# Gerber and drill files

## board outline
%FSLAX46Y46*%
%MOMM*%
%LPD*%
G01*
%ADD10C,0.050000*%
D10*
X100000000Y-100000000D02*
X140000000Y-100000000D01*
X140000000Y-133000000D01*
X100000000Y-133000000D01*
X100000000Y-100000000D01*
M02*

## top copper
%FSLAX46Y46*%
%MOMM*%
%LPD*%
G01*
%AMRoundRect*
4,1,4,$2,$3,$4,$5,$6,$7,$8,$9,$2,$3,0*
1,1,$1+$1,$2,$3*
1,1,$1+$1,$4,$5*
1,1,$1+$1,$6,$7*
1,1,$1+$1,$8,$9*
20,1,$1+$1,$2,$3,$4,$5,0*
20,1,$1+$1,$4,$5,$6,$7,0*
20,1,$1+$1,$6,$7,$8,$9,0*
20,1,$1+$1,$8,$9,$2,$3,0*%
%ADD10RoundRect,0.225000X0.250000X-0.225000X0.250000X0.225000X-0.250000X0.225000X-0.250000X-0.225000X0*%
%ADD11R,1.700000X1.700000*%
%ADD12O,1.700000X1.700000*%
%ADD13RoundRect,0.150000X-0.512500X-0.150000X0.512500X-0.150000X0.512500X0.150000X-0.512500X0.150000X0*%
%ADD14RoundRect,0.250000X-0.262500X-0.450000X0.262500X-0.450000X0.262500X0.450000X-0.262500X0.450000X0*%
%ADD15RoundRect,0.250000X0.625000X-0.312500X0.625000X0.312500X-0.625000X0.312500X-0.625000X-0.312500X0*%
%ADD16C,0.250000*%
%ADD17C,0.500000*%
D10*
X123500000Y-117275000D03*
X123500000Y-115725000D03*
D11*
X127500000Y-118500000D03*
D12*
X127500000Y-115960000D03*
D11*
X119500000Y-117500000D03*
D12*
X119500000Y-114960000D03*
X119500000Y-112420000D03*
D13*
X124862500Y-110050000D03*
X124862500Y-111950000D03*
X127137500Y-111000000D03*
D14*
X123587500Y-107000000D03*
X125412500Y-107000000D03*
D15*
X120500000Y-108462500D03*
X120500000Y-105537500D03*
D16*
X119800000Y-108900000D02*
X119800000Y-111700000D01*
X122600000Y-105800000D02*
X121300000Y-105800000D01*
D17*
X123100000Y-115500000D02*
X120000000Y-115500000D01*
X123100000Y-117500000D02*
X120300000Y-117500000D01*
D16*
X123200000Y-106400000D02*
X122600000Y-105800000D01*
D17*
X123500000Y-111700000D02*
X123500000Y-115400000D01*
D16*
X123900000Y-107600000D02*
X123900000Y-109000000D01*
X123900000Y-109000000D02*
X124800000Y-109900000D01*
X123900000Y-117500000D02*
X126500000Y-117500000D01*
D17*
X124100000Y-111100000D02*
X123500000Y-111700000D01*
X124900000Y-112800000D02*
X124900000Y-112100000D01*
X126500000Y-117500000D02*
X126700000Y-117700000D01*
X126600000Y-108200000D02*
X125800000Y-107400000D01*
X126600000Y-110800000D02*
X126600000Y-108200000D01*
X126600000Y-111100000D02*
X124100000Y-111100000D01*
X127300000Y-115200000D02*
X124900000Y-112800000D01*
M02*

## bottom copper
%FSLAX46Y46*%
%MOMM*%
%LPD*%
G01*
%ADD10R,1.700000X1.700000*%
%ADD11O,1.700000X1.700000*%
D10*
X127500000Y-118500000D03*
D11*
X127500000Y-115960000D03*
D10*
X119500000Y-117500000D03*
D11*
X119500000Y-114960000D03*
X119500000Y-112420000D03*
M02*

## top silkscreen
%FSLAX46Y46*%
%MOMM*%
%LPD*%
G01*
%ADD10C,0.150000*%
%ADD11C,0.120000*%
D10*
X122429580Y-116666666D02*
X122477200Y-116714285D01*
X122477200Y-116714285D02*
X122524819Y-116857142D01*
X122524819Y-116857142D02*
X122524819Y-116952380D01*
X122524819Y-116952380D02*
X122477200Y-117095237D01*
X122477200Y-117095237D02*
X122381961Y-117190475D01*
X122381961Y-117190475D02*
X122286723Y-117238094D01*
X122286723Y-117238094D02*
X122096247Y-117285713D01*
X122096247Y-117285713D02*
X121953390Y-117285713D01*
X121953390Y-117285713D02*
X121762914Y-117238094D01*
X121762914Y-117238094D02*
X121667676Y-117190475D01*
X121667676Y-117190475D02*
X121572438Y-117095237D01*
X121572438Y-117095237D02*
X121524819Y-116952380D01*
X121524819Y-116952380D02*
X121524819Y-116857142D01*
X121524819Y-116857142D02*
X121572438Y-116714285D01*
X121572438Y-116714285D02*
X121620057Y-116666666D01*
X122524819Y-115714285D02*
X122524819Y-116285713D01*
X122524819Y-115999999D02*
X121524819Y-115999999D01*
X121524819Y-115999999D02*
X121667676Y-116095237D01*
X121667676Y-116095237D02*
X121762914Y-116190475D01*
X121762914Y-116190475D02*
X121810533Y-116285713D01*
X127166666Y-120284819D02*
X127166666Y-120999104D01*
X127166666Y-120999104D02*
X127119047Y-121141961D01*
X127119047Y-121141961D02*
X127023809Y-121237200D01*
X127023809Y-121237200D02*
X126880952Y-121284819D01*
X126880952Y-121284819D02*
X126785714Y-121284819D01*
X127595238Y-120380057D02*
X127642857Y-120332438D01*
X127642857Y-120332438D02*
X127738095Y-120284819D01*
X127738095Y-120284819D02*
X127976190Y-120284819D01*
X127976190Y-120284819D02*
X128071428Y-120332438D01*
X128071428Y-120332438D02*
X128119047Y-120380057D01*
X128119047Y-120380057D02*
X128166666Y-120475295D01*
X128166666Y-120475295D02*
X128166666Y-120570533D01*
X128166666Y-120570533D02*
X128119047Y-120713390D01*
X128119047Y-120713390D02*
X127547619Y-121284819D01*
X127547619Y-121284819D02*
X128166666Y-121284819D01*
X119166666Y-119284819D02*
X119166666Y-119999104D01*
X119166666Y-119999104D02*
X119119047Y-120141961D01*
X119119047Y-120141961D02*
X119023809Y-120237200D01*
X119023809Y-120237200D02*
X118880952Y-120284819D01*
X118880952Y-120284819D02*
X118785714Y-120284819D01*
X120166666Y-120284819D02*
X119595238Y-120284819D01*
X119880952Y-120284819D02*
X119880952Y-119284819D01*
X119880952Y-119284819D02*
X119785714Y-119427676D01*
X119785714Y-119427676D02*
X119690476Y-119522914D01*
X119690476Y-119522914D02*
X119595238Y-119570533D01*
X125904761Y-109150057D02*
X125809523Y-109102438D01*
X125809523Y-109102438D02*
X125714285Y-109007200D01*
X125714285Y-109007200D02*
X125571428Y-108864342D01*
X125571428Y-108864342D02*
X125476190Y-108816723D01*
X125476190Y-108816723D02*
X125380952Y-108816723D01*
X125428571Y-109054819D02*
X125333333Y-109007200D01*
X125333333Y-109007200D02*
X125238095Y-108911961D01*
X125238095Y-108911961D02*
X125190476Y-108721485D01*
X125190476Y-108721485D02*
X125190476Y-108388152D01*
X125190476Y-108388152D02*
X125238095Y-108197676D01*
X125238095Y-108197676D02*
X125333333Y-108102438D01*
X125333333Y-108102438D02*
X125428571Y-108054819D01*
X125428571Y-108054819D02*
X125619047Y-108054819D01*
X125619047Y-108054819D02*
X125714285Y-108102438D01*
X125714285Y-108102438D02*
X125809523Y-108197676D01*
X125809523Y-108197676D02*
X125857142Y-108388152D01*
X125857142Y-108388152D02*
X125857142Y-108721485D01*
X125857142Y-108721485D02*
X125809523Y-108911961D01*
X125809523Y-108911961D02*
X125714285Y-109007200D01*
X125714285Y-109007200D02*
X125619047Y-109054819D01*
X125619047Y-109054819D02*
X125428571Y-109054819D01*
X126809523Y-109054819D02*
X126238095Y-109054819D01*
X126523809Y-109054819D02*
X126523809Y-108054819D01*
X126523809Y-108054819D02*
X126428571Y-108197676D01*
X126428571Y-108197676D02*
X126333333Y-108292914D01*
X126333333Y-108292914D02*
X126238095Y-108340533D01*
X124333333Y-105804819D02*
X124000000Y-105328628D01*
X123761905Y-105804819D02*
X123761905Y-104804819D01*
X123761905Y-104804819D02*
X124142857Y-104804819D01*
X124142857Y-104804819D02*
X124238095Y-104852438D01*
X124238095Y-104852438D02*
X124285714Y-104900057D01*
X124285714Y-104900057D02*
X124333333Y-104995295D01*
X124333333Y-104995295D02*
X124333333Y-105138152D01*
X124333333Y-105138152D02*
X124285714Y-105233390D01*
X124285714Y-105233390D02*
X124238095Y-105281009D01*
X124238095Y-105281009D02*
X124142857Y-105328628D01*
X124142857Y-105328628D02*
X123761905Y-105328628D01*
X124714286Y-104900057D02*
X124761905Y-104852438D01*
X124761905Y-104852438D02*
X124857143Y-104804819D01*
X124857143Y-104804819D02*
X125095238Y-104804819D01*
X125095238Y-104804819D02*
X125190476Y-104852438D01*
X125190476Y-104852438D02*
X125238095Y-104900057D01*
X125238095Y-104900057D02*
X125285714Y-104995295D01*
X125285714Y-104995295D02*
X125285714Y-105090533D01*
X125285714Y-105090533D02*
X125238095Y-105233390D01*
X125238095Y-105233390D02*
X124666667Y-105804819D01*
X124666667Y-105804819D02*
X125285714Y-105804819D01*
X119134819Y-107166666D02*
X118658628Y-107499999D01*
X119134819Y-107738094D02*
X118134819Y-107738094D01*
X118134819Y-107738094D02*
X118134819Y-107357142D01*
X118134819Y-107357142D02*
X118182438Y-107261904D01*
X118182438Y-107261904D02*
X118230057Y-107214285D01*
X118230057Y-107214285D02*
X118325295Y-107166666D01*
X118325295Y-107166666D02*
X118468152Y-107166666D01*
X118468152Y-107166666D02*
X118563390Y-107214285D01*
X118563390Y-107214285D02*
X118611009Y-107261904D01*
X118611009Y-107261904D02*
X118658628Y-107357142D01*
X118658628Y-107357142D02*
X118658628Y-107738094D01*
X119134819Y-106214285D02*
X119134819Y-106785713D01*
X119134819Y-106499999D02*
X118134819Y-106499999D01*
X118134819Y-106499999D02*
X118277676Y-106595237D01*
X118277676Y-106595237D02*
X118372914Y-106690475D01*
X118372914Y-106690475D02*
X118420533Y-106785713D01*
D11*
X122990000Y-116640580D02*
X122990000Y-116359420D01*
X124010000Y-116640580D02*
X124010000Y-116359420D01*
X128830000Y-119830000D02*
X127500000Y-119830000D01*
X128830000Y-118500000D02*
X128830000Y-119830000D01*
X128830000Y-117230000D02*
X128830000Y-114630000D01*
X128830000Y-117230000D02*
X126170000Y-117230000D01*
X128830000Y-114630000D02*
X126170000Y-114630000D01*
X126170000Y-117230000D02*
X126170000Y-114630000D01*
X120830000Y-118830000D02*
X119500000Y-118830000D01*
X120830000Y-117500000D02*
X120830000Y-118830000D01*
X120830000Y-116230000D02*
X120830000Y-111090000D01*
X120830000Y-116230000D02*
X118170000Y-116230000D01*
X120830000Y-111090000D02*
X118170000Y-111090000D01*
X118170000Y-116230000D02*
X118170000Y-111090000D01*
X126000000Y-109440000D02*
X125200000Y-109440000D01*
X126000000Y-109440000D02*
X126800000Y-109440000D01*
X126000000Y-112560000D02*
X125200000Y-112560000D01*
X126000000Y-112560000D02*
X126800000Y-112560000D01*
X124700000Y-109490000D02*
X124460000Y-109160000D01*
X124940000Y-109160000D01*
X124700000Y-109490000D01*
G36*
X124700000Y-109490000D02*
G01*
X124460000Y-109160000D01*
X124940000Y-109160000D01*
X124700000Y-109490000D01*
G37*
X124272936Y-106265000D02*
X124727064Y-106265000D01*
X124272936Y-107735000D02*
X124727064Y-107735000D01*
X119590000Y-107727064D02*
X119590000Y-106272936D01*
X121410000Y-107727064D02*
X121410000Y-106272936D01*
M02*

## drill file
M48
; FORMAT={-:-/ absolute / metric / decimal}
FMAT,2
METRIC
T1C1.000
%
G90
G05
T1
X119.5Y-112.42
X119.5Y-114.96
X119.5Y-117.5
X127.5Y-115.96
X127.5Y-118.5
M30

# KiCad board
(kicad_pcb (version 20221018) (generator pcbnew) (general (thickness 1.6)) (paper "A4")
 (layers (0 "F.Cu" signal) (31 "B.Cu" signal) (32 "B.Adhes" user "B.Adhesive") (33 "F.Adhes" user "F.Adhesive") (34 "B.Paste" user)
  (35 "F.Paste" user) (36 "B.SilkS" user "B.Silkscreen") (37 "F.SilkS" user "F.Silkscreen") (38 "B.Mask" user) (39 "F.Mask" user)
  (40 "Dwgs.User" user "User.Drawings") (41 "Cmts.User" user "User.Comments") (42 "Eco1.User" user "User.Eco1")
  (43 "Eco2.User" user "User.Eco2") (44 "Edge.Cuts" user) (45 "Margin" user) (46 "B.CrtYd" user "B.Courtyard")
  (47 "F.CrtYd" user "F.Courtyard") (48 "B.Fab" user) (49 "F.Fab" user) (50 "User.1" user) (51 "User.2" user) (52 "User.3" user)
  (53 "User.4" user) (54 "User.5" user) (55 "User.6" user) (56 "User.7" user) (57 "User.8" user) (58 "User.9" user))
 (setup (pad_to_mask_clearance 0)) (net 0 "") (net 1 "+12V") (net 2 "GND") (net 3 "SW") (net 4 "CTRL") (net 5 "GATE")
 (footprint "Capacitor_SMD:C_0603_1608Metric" (layer "F.Cu") (at 123.5 116.5 90)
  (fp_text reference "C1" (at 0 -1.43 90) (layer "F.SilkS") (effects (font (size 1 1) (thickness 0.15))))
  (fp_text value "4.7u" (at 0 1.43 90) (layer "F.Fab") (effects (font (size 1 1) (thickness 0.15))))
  (fp_line (start -0.14058 -0.51) (end 0.14058 -0.51) (stroke (width 0.12) (type solid)) (layer "F.SilkS"))
  (fp_line (start -0.14058 0.51) (end 0.14058 0.51) (stroke (width 0.12) (type solid)) (layer "F.SilkS"))
  (pad "1" smd roundrect (at -0.775 0 90) (size 0.9 0.95) (layers "F.Cu" "F.Paste" "F.Mask") (roundrect_rratio 0.25) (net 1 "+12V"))
  (pad "2" smd roundrect (at 0.775 0 90) (size 0.9 0.95) (layers "F.Cu" "F.Paste" "F.Mask") (roundrect_rratio 0.25) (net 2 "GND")))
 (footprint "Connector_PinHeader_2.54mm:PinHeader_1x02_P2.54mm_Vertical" (layer "F.Cu") (at 127.5 118.5 180)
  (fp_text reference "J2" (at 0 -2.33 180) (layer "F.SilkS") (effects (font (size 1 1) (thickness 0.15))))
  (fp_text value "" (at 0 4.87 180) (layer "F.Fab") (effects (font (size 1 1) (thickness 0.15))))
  (fp_line (start -1.33 -1.33) (end 0 -1.33) (stroke (width 0.12) (type solid)) (layer "F.SilkS"))
  (fp_line (start -1.33 0) (end -1.33 -1.33) (stroke (width 0.12) (type solid)) (layer "F.SilkS"))
  (fp_line (start -1.33 1.27) (end -1.33 3.87) (stroke (width 0.12) (type solid)) (layer "F.SilkS"))
  (fp_line (start -1.33 1.27) (end 1.33 1.27) (stroke (width 0.12) (type solid)) (layer "F.SilkS"))
  (fp_line (start -1.33 3.87) (end 1.33 3.87) (stroke (width 0.12) (type solid)) (layer "F.SilkS"))
  (fp_line (start 1.33 1.27) (end 1.33 3.87) (stroke (width 0.12) (type solid)) (layer "F.SilkS"))
  (pad "1" thru_hole rect (at 0 0 180) (size 1.7 1.7) (drill 1) (layers "*.Cu" "*.Mask") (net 1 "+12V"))
  (pad "2" thru_hole oval (at 0 2.54 180) (size 1.7 1.7) (drill 1) (layers "*.Cu" "*.Mask") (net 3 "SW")))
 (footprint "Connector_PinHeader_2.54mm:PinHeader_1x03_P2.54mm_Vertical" (layer "F.Cu") (at 119.5 117.5 180)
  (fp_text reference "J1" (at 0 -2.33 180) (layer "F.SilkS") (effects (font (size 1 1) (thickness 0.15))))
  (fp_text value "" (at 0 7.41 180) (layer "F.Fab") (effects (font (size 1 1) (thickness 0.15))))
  (fp_line (start -1.33 -1.33) (end 0 -1.33) (stroke (width 0.12) (type solid)) (layer "F.SilkS"))
  (fp_line (start -1.33 0) (end -1.33 -1.33) (stroke (width 0.12) (type solid)) (layer "F.SilkS"))
  (fp_line (start -1.33 1.27) (end -1.33 6.41) (stroke (width 0.12) (type solid)) (layer "F.SilkS"))
  (fp_line (start -1.33 1.27) (end 1.33 1.27) (stroke (width 0.12) (type solid)) (layer "F.SilkS"))
  (fp_line (start -1.33 6.41) (end 1.33 6.41) (stroke (width 0.12) (type solid)) (layer "F.SilkS"))
  (fp_line (start 1.33 1.27) (end 1.33 6.41) (stroke (width 0.12) (type solid)) (layer "F.SilkS"))
  (pad "1" thru_hole rect (at 0 0 180) (size 1.7 1.7) (drill 1) (layers "*.Cu" "*.Mask") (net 1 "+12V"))
  (pad "2" thru_hole oval (at 0 2.54 180) (size 1.7 1.7) (drill 1) (layers "*.Cu" "*.Mask") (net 2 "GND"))
  (pad "3" thru_hole oval (at 0 5.08 180) (size 1.7 1.7) (drill 1) (layers "*.Cu" "*.Mask") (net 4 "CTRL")))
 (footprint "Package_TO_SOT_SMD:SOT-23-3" (layer "F.Cu") (at 126 111)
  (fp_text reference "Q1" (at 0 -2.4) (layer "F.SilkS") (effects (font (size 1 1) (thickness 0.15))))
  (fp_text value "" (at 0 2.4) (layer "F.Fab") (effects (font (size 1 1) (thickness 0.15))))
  (fp_line (start 0 -1.56) (end -0.8 -1.56) (stroke (width 0.12) (type solid)) (layer "F.SilkS"))
  (fp_line (start 0 -1.56) (end 0.8 -1.56) (stroke (width 0.12) (type solid)) (layer "F.SilkS"))
  (fp_line (start 0 1.56) (end -0.8 1.56) (stroke (width 0.12) (type solid)) (layer "F.SilkS"))
  (fp_line (start 0 1.56) (end 0.8 1.56) (stroke (width 0.12) (type solid)) (layer "F.SilkS"))
  (fp_poly
   (pts (xy -1.3 -1.51) (xy -1.54 -1.84) (xy -1.06 -1.84) (xy -1.3 -1.51)) (stroke (width 0.12) (type solid)) (fill solid) (layer "F.SilkS"))
  (pad "1" smd roundrect (at -1.1375 -0.95) (size 1.325 0.6) (layers "F.Cu" "F.Paste" "F.Mask") (roundrect_rratio 0.25) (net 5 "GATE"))
  (pad "2" smd roundrect (at -1.1375 0.95) (size 1.325 0.6) (layers "F.Cu" "F.Paste" "F.Mask") (roundrect_rratio 0.25) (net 3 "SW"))
  (pad "3" smd roundrect (at 1.1375 0) (size 1.325 0.6) (layers "F.Cu" "F.Paste" "F.Mask") (roundrect_rratio 0.25) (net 2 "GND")))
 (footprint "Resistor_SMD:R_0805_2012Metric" (layer "F.Cu") (at 124.5 107)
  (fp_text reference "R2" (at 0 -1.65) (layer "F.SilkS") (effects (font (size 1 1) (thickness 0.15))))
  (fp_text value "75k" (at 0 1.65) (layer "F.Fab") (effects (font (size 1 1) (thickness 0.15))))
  (fp_line (start -0.227064 -0.735) (end 0.227064 -0.735) (stroke (width 0.12) (type solid)) (layer "F.SilkS"))
  (fp_line (start -0.227064 0.735) (end 0.227064 0.735) (stroke (width 0.12) (type solid)) (layer "F.SilkS"))
  (pad "1" smd roundrect (at -0.9125 0) (size 1.025 1.4) (layers "F.Cu" "F.Paste" "F.Mask") (roundrect_rratio 0.243902) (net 5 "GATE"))
  (pad "2" smd roundrect (at 0.9125 0) (size 1.025 1.4) (layers "F.Cu" "F.Paste" "F.Mask") (roundrect_rratio 0.243902) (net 2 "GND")))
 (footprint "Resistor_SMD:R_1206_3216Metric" (layer "F.Cu") (at 120.5 107 90)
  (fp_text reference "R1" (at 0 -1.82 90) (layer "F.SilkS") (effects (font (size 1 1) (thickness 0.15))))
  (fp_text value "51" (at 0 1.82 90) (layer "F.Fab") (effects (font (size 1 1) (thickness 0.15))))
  (fp_line (start -0.727064 -0.91) (end 0.727064 -0.91) (stroke (width 0.12) (type solid)) (layer "F.SilkS"))
  (fp_line (start -0.727064 0.91) (end 0.727064 0.91) (stroke (width 0.12) (type solid)) (layer "F.SilkS"))
  (pad "1" smd roundrect (at -1.4625 0 90) (size 1.125 1.75) (layers "F.Cu" "F.Paste" "F.Mask") (roundrect_rratio 0.222222) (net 4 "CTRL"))
  (pad "2" smd roundrect (at 1.4625 0 90) (size 1.125 1.75) (layers "F.Cu" "F.Paste" "F.Mask") (roundrect_rratio 0.222222) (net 5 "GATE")))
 (gr_rect (start 100 100) (end 140 133) (stroke (width 0.05) (type default)) (fill none) (layer "Edge.Cuts"))
 (segment (start 119.8 108.9) (end 119.8 111.7) (width 0.25) (layer "F.Cu") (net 4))
 (segment (start 122.6 105.8) (end 121.3 105.8) (width 0.25) (layer "F.Cu") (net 5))
 (segment (start 123.1 115.5) (end 120 115.5) (width 0.5) (layer "F.Cu") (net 2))
 (segment (start 123.1 117.5) (end 120.3 117.5) (width 0.5) (layer "F.Cu") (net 1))
 (segment (start 123.2 106.4) (end 122.6 105.8) (width 0.25) (layer "F.Cu") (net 5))
 (segment (start 123.5 111.7) (end 123.5 115.4) (width 0.5) (layer "F.Cu") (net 2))
 (segment (start 123.9 107.6) (end 123.9 109) (width 0.25) (layer "F.Cu") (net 5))
 (segment (start 123.9 109) (end 124.8 109.9) (width 0.25) (layer "F.Cu") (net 5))
 (segment (start 123.9 117.5) (end 126.5 117.5) (width 0.25) (layer "F.Cu") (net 1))
 (segment (start 124.1 111.1) (end 123.5 111.7) (width 0.5) (layer "F.Cu") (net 2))
 (segment (start 124.9 112.8) (end 124.9 112.1) (width 0.5) (layer "F.Cu") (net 3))
 (segment (start 126.5 117.5) (end 126.7 117.7) (width 0.5) (layer "F.Cu") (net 1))
 (segment (start 126.6 108.2) (end 125.8 107.4) (width 0.5) (layer "F.Cu") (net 2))
 (segment (start 126.6 110.8) (end 126.6 108.2) (width 0.5) (layer "F.Cu") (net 2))
 (segment (start 126.6 111.1) (end 124.1 111.1) (width 0.5) (layer "F.Cu") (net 2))
 (segment (start 127.3 115.2) (end 124.9 112.8) (width 0.5) (layer "F.Cu") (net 3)))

